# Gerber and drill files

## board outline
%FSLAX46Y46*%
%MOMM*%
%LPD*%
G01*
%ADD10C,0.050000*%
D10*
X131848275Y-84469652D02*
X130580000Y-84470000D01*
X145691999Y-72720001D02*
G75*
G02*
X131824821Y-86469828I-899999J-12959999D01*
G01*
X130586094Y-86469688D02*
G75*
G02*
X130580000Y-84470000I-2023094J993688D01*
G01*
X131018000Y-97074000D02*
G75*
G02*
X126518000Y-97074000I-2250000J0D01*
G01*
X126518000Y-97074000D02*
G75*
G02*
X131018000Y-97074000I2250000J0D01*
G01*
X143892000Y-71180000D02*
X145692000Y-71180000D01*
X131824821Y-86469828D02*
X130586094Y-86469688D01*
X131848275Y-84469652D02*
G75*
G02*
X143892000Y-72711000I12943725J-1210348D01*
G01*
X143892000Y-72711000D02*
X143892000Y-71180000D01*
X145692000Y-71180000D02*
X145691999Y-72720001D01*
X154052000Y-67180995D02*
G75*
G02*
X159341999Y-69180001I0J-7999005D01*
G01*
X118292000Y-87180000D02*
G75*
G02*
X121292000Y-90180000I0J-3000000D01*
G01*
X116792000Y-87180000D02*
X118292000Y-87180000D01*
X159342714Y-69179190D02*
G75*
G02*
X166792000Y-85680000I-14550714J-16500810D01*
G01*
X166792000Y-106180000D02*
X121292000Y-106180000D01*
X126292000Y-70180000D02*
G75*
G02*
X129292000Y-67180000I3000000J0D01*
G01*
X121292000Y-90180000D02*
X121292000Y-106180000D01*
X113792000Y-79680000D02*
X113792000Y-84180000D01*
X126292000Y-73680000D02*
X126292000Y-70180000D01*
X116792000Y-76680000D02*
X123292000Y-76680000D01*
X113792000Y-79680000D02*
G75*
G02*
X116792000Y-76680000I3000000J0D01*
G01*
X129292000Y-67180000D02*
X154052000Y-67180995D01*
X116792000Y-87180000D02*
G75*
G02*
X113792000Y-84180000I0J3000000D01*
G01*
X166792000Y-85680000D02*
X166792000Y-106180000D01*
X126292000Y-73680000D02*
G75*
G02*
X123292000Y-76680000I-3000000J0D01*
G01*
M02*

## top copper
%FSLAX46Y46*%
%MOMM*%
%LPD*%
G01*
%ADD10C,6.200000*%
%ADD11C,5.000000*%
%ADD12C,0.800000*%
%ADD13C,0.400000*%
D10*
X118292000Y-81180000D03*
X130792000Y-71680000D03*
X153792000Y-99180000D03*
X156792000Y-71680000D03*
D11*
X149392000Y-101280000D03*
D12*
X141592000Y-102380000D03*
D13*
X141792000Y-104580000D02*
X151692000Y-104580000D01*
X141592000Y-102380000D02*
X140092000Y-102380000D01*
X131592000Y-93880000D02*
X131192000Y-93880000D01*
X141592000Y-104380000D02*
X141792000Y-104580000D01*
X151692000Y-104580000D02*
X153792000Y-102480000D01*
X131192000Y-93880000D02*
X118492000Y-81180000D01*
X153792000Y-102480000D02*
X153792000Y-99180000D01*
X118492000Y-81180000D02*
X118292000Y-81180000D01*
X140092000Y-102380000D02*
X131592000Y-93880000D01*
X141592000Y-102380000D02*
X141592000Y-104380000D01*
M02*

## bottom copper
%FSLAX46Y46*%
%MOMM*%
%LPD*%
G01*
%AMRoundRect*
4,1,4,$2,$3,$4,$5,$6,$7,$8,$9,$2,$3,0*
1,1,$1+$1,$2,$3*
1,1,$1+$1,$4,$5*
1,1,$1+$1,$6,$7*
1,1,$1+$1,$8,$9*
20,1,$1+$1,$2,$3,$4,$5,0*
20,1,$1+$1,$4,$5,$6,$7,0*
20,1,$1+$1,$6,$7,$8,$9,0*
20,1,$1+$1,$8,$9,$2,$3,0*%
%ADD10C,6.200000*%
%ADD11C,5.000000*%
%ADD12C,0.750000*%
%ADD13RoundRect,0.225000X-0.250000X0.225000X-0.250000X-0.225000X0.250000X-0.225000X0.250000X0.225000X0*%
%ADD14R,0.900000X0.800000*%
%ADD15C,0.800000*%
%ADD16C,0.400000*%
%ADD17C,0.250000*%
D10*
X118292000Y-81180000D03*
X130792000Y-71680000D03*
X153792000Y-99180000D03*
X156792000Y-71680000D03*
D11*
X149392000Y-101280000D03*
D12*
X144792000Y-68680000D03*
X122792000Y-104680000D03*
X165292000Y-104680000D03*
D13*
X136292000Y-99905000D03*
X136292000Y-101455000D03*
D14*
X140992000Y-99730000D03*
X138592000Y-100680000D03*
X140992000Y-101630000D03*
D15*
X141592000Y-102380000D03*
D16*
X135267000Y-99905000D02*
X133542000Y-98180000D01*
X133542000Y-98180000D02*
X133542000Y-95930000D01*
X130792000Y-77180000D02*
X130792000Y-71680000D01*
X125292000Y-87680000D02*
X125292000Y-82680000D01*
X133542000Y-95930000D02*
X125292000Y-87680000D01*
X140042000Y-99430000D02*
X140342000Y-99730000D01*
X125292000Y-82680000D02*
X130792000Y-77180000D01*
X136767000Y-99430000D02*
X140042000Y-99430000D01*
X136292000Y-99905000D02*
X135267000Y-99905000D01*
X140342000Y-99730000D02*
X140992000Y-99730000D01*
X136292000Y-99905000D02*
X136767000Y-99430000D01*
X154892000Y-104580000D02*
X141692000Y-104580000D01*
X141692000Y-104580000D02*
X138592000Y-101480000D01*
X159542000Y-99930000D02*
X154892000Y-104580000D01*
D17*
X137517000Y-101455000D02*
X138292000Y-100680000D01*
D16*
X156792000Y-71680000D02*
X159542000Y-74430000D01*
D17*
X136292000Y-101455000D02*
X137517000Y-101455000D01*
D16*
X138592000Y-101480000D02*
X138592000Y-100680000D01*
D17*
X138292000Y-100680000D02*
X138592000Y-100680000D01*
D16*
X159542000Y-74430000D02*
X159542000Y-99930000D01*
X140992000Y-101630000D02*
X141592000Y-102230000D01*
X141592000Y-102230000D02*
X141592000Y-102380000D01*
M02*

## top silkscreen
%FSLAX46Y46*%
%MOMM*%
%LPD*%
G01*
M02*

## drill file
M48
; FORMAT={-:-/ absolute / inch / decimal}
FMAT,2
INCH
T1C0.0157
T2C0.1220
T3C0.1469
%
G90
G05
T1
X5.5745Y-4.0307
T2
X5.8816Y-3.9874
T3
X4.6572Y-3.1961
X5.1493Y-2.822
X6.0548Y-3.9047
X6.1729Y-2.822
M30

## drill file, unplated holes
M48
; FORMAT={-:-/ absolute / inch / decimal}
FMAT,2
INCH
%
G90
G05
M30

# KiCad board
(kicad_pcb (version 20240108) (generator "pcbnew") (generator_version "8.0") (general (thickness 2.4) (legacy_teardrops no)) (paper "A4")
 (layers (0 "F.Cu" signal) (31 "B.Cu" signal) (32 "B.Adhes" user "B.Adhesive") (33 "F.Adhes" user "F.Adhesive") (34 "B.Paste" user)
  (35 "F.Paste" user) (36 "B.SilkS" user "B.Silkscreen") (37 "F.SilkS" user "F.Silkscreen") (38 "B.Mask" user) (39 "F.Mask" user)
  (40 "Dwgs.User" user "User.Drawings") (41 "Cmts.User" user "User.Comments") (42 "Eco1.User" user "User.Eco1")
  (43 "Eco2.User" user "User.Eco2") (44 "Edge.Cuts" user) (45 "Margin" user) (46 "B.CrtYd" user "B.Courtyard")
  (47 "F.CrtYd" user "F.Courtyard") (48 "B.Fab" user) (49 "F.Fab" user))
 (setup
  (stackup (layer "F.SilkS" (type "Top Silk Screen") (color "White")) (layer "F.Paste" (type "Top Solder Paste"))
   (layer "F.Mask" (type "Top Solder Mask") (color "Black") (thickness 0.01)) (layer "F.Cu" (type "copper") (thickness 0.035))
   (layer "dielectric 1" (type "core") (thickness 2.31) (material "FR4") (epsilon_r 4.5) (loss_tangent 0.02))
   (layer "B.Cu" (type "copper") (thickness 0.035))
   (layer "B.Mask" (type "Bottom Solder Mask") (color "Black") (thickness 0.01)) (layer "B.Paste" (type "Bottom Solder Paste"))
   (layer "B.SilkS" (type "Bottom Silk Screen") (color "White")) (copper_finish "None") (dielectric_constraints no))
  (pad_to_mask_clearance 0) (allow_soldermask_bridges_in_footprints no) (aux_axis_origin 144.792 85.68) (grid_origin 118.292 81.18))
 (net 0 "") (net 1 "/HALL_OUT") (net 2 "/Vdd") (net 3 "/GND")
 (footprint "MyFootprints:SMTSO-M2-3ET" (layer "F.Cu") (at 118.292 81.18 180)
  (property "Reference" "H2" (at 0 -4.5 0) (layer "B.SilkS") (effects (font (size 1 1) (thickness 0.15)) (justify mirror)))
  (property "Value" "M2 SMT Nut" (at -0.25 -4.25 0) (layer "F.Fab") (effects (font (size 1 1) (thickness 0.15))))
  (pad "1" thru_hole circle (at 0 0 180) (size 6.2 6.2) (drill 3.73) (layers "*.Cu" "*.Mask" "B.Paste") (remove_unused_layers no)
   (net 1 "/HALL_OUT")))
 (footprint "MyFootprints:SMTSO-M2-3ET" (layer "F.Cu") (at 130.792 71.68 180)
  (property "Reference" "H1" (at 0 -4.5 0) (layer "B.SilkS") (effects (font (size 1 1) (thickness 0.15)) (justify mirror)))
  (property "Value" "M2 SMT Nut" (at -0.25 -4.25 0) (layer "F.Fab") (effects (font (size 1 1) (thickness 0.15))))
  (pad "1" thru_hole circle (at 0 0 180) (size 6.2 6.2) (drill 3.73) (layers "*.Cu" "*.Mask" "B.Paste") (remove_unused_layers no)
   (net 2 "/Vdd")))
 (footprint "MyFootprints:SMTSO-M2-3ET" (layer "F.Cu") (at 153.792 99.18 180)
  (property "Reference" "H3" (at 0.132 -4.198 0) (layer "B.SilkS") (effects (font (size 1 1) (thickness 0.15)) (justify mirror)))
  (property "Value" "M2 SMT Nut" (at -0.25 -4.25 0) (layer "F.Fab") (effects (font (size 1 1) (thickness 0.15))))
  (pad "1" thru_hole circle (at 0 0 180) (size 6.2 6.2) (drill 3.73) (layers "*.Cu" "*.Mask" "B.Paste") (remove_unused_layers no)
   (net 1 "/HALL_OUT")))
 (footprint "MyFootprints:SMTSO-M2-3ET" (layer "F.Cu") (at 156.792 71.68 180)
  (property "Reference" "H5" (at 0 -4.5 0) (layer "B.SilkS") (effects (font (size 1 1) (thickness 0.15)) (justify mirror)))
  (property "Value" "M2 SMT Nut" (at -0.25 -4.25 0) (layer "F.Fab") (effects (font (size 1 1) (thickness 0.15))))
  (pad "1" thru_hole circle (at 0 0 180) (size 6.2 6.2) (drill 3.73) (layers "*.Cu" "*.Mask" "B.Paste") (remove_unused_layers no)
   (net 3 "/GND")))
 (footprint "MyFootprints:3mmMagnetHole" (layer "F.Cu") (at 149.392 101.28)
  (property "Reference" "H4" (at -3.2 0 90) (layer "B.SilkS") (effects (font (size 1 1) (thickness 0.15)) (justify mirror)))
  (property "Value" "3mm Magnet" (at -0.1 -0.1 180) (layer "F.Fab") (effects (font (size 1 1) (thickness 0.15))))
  (pad "1" thru_hole circle (at 0 0) (size 5 5) (drill 3.1) (layers "*.Cu" "*.Mask" "F.Paste") (remove_unused_layers no)))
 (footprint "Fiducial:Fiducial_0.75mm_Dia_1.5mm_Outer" (layer "B.Cu") (at 144.792 68.68)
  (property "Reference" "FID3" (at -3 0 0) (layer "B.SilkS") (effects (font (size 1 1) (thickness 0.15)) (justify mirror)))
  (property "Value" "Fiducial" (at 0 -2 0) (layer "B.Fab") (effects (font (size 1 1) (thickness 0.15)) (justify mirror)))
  (pad "" smd circle (at 0 0) (size 0.75 0.75) (layers "B.Cu" "B.Mask") (solder_mask_margin 0.375) (clearance 0.375)))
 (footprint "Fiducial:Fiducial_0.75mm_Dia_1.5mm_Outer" (layer "B.Cu") (at 122.792 104.68)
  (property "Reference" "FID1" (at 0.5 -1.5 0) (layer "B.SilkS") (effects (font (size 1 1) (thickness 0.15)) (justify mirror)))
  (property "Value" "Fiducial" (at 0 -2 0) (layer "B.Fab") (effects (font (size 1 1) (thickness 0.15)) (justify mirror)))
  (pad "" smd circle (at 0 0) (size 0.75 0.75) (layers "B.Cu" "B.Mask") (solder_mask_margin 0.375) (clearance 0.375)))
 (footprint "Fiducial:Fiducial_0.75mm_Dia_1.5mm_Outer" (layer "B.Cu") (at 165.292 104.68)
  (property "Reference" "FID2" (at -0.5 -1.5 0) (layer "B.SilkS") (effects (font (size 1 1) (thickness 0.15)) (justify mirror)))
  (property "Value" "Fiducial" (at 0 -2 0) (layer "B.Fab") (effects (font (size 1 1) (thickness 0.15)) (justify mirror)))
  (pad "" smd circle (at 0 0) (size 0.75 0.75) (layers "B.Cu" "B.Mask") (solder_mask_margin 0.375) (clearance 0.375)))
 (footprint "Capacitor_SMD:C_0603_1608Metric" (layer "B.Cu") (at 136.292 100.68 -90)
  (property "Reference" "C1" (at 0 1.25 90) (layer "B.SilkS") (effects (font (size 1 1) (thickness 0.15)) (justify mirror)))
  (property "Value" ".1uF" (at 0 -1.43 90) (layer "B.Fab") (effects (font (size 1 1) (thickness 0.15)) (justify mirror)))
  (pad "1" smd roundrect (at -0.775 0 270) (size 0.9 0.95) (layers "B.Cu" "B.Paste" "B.Mask") (roundrect_rratio 0.25) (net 2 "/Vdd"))
  (pad "2" smd roundrect (at 0.775 0 270) (size 0.9 0.95) (layers "B.Cu" "B.Paste" "B.Mask") (roundrect_rratio 0.25) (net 3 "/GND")))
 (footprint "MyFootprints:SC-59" (layer "B.Cu") (at 139.792 100.68)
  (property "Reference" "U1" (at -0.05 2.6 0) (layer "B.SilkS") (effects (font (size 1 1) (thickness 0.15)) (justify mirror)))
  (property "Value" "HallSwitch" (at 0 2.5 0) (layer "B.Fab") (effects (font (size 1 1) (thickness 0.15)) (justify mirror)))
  (pad "1" smd rect (at 1.2 -0.95 180) (size 0.9 0.8) (layers "B.Cu" "B.Paste" "B.Mask") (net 2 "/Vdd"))
  (pad "2" smd rect (at -1.2 0 180) (size 0.9 0.8) (layers "B.Cu" "B.Paste" "B.Mask") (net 3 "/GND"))
  (pad "3" smd rect (at 1.2 0.95 180) (size 0.9 0.8) (layers "B.Cu" "B.Paste" "B.Mask") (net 1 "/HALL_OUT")))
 (gr_line (start 131.848275 84.469652) (end 130.58 84.47) (stroke (width 0.05) (type solid)) (layer "Edge.Cuts"))
 (gr_arc (start 145.691999 72.720001) (mid 153.939058 94.905124) (end 131.824821 86.469828) (stroke (width 0.05) (type solid))
  (layer "Edge.Cuts"))
 (gr_arc (start 130.586094 86.469688) (mid 126.309053 85.482869) (end 130.58 84.47) (stroke (width 0.05) (type solid)) (layer "Edge.Cuts"))
 (gr_circle (center 128.768 97.074) (end 131.018 97.074) (stroke (width 0.05) (type solid)) (fill none) (layer "Edge.Cuts"))
 (gr_line (start 143.892 71.18) (end 145.692 71.18) (stroke (width 0.05) (type solid)) (layer "Edge.Cuts"))
 (gr_line (start 131.824821 86.469828) (end 130.586094 86.469688) (stroke (width 0.05) (type solid)) (layer "Edge.Cuts"))
 (gr_arc (start 131.848275 84.469652) (mid 135.710224 76.378048) (end 143.892 72.711) (stroke (width 0.05) (type solid)) (layer "Edge.Cuts"))
 (gr_line (start 143.892 72.711) (end 143.892 71.18) (stroke (width 0.05) (type solid)) (layer "Edge.Cuts"))
 (gr_line (start 145.692 71.18) (end 145.691999 72.720001) (stroke (width 0.05) (type solid)) (layer "Edge.Cuts"))
 (gr_arc (start 154.052 67.180995) (mid 156.879548 67.697417) (end 159.341999 69.180001) (stroke (width 0.05) (type solid))
  (layer "Edge.Cuts"))
 (gr_arc (start 118.292 87.18) (mid 120.41332 88.05868) (end 121.292 90.18) (stroke (width 0.05) (type solid)) (layer "Edge.Cuts"))
 (gr_line (start 116.792 87.18) (end 118.292 87.18) (stroke (width 0.05) (type solid)) (layer "Edge.Cuts"))
 (gr_arc (start 159.342714 69.17919) (mid 164.84338 76.62781) (end 166.792 85.68) (stroke (width 0.05) (type solid)) (layer "Edge.Cuts"))
 (gr_line (start 166.792 106.18) (end 121.292 106.18) (stroke (width 0.05) (type solid)) (layer "Edge.Cuts"))
 (gr_arc (start 126.292 70.18) (mid 127.17068 68.05868) (end 129.292 67.18) (stroke (width 0.05) (type solid)) (layer "Edge.Cuts"))
 (gr_line (start 121.292 90.18) (end 121.292 106.18) (stroke (width 0.05) (type solid)) (layer "Edge.Cuts"))
 (gr_line (start 113.792 79.68) (end 113.792 84.18) (stroke (width 0.05) (type solid)) (layer "Edge.Cuts"))
 (gr_line (start 126.292 73.68) (end 126.292 70.18) (stroke (width 0.05) (type solid)) (layer "Edge.Cuts"))
 (gr_line (start 116.792 76.68) (end 123.292 76.68) (stroke (width 0.05) (type solid)) (layer "Edge.Cuts"))
 (gr_arc (start 113.792 79.68) (mid 114.67068 77.55868) (end 116.792 76.68) (stroke (width 0.05) (type solid)) (layer "Edge.Cuts"))
 (gr_line (start 129.292 67.18) (end 154.052 67.180995) (stroke (width 0.05) (type solid)) (layer "Edge.Cuts"))
 (gr_arc (start 116.792 87.18) (mid 114.67068 86.30132) (end 113.792 84.18) (stroke (width 0.05) (type solid)) (layer "Edge.Cuts"))
 (gr_line (start 166.792 85.68) (end 166.792 106.18) (stroke (width 0.05) (type solid)) (layer "Edge.Cuts"))
 (gr_arc (start 126.292 73.68) (mid 125.41332 75.80132) (end 123.292 76.68) (stroke (width 0.05) (type solid)) (layer "Edge.Cuts"))
 (segment (start 135.267 99.905) (end 133.542 98.18) (width 0.4) (layer "B.Cu") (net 2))
 (segment (start 133.542 98.18) (end 133.542 95.93) (width 0.4) (layer "B.Cu") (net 2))
 (segment (start 130.792 77.18) (end 130.792 71.68) (width 0.4) (layer "B.Cu") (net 2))
 (segment (start 125.292 87.68) (end 125.292 82.68) (width 0.4) (layer "B.Cu") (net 2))
 (segment (start 133.542 95.93) (end 125.292 87.68) (width 0.4) (layer "B.Cu") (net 2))
 (segment (start 140.042 99.43) (end 140.342 99.73) (width 0.4) (layer "B.Cu") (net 2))
 (segment (start 125.292 82.68) (end 130.792 77.18) (width 0.4) (layer "B.Cu") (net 2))
 (segment (start 136.767 99.43) (end 140.042 99.43) (width 0.4) (layer "B.Cu") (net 2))
 (segment (start 136.292 99.905) (end 135.267 99.905) (width 0.4) (layer "B.Cu") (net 2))
 (segment (start 140.342 99.73) (end 140.992 99.73) (width 0.4) (layer "B.Cu") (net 2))
 (segment (start 136.292 99.905) (end 136.767 99.43) (width 0.4) (layer "B.Cu") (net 2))
 (segment (start 154.892 104.58) (end 141.692 104.58) (width 0.4) (layer "B.Cu") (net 3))
 (segment (start 141.692 104.58) (end 138.592 101.48) (width 0.4) (layer "B.Cu") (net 3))
 (segment (start 159.542 99.93) (end 154.892 104.58) (width 0.4) (layer "B.Cu") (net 3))
 (segment (start 137.517 101.455) (end 138.292 100.68) (width 0.25) (layer "B.Cu") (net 3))
 (segment (start 156.792 71.68) (end 159.542 74.43) (width 0.4) (layer "B.Cu") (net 3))
 (segment (start 136.292 101.455) (end 137.517 101.455) (width 0.25) (layer "B.Cu") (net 3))
 (segment (start 138.592 101.48) (end 138.592 100.68) (width 0.4) (layer "B.Cu") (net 3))
 (segment (start 138.292 100.68) (end 138.592 100.68) (width 0.25) (layer "B.Cu") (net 3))
 (segment (start 159.542 74.43) (end 159.542 99.93) (width 0.4) (layer "B.Cu") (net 3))
 (segment (start 141.792 104.58) (end 151.692 104.58) (width 0.4) (layer "F.Cu") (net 1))
 (segment (start 141.592 102.38) (end 140.092 102.38) (width 0.4) (layer "F.Cu") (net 1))
 (segment (start 131.592 93.88) (end 131.192 93.88) (width 0.4) (layer "F.Cu") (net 1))
 (segment (start 141.592 104.38) (end 141.792 104.58) (width 0.4) (layer "F.Cu") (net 1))
 (segment (start 151.692 104.58) (end 153.792 102.48) (width 0.4) (layer "F.Cu") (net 1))
 (segment (start 131.192 93.88) (end 118.492 81.18) (width 0.4) (layer "F.Cu") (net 1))
 (segment (start 153.792 102.48) (end 153.792 99.18) (width 0.4) (layer "F.Cu") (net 1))
 (segment (start 118.492 81.18) (end 118.292 81.18) (width 0.4) (layer "F.Cu") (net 1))
 (segment (start 140.092 102.38) (end 131.592 93.88) (width 0.4) (layer "F.Cu") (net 1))
 (segment (start 141.592 102.38) (end 141.592 104.38) (width 0.4) (layer "F.Cu") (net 1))
 (via (at 141.592 102.38) (size 0.8) (drill 0.4) (layers "F.Cu" "B.Cu") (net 1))
 (segment (start 140.992 101.63) (end 141.592 102.23) (width 0.4) (layer "B.Cu") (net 1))
 (segment (start 141.592 102.23) (end 141.592 102.38) (width 0.4) (layer "B.Cu") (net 1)))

